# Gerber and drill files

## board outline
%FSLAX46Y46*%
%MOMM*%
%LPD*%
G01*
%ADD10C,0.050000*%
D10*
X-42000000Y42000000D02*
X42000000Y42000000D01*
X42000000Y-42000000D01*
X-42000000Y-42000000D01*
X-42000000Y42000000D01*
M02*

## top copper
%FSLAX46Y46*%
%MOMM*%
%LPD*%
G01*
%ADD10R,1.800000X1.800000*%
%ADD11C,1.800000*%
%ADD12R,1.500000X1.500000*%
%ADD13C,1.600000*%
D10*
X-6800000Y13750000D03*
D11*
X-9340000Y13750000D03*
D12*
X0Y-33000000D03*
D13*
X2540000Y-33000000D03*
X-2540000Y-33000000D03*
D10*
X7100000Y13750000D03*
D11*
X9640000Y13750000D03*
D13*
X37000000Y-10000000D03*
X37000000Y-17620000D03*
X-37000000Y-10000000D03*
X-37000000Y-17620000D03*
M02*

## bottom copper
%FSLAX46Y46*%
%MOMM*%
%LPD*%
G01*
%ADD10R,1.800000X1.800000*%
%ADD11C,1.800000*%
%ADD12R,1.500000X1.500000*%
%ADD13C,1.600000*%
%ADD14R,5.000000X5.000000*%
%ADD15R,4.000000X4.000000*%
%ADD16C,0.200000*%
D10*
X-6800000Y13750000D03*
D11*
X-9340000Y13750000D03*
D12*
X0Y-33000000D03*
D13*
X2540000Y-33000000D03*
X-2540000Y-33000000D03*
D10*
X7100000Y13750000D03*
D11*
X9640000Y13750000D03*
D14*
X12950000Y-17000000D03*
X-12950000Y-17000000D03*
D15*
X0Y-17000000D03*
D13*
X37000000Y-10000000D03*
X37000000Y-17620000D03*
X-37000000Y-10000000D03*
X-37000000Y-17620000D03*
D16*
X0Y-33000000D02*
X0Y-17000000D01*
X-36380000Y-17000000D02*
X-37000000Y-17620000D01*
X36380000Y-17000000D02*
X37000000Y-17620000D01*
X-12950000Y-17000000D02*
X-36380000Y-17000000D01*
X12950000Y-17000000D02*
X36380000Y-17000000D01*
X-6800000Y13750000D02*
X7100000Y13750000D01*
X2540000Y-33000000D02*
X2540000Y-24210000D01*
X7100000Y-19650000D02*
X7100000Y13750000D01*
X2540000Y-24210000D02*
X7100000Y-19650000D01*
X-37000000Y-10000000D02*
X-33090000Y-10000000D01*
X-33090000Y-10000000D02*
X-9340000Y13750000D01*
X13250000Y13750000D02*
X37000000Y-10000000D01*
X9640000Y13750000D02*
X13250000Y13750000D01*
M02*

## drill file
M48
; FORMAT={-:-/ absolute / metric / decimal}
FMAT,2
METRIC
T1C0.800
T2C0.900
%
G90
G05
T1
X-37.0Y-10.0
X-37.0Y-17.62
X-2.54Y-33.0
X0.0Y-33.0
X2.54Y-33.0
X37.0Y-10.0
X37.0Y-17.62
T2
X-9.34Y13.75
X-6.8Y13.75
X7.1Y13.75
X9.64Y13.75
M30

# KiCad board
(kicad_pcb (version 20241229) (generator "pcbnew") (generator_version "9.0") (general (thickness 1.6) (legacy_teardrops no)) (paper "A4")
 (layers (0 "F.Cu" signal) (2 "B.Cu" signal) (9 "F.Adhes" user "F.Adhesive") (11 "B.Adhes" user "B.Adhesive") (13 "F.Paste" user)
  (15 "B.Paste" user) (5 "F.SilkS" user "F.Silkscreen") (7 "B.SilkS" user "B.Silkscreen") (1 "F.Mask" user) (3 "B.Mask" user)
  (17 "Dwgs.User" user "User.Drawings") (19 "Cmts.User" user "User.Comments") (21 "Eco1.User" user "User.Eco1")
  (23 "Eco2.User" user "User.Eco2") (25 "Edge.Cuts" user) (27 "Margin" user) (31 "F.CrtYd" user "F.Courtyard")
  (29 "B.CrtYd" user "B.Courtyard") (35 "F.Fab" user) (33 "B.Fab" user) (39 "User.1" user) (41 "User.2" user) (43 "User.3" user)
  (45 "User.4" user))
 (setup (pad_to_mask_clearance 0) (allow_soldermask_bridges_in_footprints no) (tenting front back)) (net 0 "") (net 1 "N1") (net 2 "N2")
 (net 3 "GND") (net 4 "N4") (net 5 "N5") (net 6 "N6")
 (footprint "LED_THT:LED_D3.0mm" (layer "F.Cu") (at -6.8 -13.75 180)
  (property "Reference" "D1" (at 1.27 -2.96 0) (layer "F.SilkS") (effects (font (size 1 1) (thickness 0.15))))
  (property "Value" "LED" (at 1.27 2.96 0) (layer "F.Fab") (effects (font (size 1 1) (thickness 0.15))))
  (pad "1" thru_hole rect (at 0 0 180) (size 1.8 1.8) (drill 0.9) (layers "*.Cu" "*.Mask") (remove_unused_layers no) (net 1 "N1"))
  (pad "2" thru_hole circle (at 2.54 0 180) (size 1.8 1.8) (drill 0.9) (layers "*.Cu" "*.Mask") (remove_unused_layers no) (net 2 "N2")))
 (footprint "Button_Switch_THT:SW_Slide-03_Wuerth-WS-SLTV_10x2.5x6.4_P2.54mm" (layer "F.Cu") (at 0 33 180)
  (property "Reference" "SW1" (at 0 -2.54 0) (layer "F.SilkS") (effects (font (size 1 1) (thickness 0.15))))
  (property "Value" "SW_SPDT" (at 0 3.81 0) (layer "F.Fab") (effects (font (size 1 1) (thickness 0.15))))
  (pad "1" thru_hole rect (at 0 0 180) (size 1.5 1.5) (drill 0.8) (layers "*.Cu" "*.Mask") (remove_unused_layers no) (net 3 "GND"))
  (pad "2" thru_hole circle (at -2.54 0 180) (size 1.6 1.6) (drill 0.8) (layers "*.Cu" "*.Mask") (remove_unused_layers no) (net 1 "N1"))
  (pad "3" thru_hole circle (at 2.54 0 180) (size 1.6 1.6) (drill 0.8) (layers "*.Cu" "*.Mask") (remove_unused_layers no) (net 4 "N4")))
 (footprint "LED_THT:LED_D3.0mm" (layer "F.Cu") (at 7.1 -13.75)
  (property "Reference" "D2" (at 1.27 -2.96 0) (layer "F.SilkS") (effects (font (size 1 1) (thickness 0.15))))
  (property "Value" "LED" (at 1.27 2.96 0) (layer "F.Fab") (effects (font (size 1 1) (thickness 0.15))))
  (pad "1" thru_hole rect (at 0 0) (size 1.8 1.8) (drill 0.9) (layers "*.Cu" "*.Mask") (remove_unused_layers no) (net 1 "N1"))
  (pad "2" thru_hole circle (at 2.54 0) (size 1.8 1.8) (drill 0.9) (layers "*.Cu" "*.Mask") (remove_unused_layers no) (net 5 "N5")))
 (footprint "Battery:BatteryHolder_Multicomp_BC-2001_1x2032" (layer "B.Cu") (at 0 17 180)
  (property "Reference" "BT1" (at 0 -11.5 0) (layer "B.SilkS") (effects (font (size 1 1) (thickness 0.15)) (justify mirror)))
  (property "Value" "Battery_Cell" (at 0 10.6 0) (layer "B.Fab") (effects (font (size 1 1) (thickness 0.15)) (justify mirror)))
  (pad "1" smd rect (at -12.95 0 180) (size 5 5) (layers "B.Cu" "B.Mask" "B.Paste") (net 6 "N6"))
  (pad "1" smd rect (at 12.95 0 180) (size 5 5) (layers "B.Cu" "B.Mask" "B.Paste") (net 6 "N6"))
  (pad "2" smd rect (at 0 0 180) (size 4 4) (layers "B.Cu" "B.Mask" "B.Paste") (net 3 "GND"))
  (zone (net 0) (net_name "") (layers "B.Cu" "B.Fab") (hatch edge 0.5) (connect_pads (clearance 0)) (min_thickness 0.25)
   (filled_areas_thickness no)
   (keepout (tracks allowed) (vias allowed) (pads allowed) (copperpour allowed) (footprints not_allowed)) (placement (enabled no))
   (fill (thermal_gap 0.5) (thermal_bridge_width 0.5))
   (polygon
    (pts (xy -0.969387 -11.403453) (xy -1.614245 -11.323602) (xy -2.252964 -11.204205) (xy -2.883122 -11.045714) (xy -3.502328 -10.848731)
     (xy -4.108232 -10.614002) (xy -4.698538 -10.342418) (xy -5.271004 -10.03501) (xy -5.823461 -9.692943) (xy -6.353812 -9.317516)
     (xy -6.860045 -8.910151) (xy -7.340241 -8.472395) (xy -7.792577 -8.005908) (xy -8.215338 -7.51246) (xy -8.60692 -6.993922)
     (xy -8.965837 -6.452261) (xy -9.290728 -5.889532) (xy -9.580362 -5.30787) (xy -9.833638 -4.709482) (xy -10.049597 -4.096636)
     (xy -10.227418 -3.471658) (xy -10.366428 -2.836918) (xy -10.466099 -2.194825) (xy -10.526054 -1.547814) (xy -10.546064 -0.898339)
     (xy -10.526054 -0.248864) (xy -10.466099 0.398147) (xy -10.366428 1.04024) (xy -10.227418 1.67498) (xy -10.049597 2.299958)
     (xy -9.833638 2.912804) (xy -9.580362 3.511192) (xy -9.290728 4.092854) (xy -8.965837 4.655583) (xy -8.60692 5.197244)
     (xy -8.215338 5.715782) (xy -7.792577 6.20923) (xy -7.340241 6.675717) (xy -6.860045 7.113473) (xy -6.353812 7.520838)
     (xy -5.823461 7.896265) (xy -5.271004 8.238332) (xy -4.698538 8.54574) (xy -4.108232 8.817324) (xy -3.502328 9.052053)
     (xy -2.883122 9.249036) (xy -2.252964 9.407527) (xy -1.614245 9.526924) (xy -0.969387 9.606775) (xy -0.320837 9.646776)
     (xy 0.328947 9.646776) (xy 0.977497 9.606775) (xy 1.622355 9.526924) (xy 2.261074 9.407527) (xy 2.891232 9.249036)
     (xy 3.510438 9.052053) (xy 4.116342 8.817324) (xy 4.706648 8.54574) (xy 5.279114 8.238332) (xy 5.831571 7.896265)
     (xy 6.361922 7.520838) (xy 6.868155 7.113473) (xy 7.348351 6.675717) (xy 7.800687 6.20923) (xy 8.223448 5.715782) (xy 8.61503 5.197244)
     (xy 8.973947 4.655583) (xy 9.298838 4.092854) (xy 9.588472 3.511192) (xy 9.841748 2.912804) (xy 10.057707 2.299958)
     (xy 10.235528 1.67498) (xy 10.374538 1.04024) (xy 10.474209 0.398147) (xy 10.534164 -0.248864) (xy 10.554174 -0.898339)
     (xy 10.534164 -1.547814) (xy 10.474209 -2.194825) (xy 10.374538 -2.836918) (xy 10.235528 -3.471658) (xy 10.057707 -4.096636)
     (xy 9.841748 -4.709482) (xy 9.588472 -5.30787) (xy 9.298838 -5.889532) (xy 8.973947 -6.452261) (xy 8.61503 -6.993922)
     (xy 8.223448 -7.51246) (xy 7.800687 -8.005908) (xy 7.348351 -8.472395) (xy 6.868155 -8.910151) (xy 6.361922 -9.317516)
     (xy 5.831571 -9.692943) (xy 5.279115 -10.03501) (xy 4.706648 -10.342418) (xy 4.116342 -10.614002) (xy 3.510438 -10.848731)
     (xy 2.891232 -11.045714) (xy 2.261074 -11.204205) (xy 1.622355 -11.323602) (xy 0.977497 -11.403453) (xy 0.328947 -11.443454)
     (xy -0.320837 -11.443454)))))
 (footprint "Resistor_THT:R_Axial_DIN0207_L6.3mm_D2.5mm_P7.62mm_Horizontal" (layer "B.Cu") (at 37 10 -90)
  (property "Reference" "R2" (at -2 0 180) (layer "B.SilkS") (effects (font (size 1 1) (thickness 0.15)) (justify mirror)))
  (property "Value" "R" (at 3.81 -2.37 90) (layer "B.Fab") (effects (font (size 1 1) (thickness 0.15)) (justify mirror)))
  (pad "1" thru_hole circle (at 0 0 270) (size 1.6 1.6) (drill 0.8) (layers "*.Cu" "*.Mask") (remove_unused_layers no) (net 5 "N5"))
  (pad "2" thru_hole circle (at 7.62 0 270) (size 1.6 1.6) (drill 0.8) (layers "*.Cu" "*.Mask") (remove_unused_layers no) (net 6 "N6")))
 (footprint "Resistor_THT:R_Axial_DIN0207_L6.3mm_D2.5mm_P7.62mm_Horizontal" (layer "B.Cu") (at -37 10 -90)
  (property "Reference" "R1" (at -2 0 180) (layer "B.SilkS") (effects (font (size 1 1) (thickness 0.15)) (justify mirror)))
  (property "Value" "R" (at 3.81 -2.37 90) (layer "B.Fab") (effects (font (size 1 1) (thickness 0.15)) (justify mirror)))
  (pad "1" thru_hole circle (at 0 0 270) (size 1.6 1.6) (drill 0.8) (layers "*.Cu" "*.Mask") (remove_unused_layers no) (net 2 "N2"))
  (pad "2" thru_hole circle (at 7.62 0 270) (size 1.6 1.6) (drill 0.8) (layers "*.Cu" "*.Mask") (remove_unused_layers no) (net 6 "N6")))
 (gr_rect (start -42 -42) (end 42 42) (stroke (width 0.05) (type solid)) (fill no) (layer "Edge.Cuts"))
 (segment (start 0 33) (end 0 17) (width 0.2) (layer "B.Cu") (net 3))
 (segment (start -36.38 17) (end -37 17.62) (width 0.2) (layer "B.Cu") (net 6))
 (segment (start 36.38 17) (end 37 17.62) (width 0.2) (layer "B.Cu") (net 6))
 (segment (start -12.95 17) (end -36.38 17) (width 0.2) (layer "B.Cu") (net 6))
 (segment (start 12.95 17) (end 36.38 17) (width 0.2) (layer "B.Cu") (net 6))
 (segment (start -6.8 -13.75) (end 7.1 -13.75) (width 0.2) (layer "B.Cu") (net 1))
 (segment (start 2.54 33) (end 2.54 24.21) (width 0.2) (layer "B.Cu") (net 1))
 (segment (start 7.1 19.65) (end 7.1 -13.75) (width 0.2) (layer "B.Cu") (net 1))
 (segment (start 2.54 24.21) (end 7.1 19.65) (width 0.2) (layer "B.Cu") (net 1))
 (segment (start -37 10) (end -33.09 10) (width 0.2) (layer "B.Cu") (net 2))
 (segment (start -33.09 10) (end -9.34 -13.75) (width 0.2) (layer "B.Cu") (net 2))
 (segment (start 13.25 -13.75) (end 37 10) (width 0.2) (layer "B.Cu") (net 5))
 (segment (start 9.64 -13.75) (end 13.25 -13.75) (width 0.2) (layer "B.Cu") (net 5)))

